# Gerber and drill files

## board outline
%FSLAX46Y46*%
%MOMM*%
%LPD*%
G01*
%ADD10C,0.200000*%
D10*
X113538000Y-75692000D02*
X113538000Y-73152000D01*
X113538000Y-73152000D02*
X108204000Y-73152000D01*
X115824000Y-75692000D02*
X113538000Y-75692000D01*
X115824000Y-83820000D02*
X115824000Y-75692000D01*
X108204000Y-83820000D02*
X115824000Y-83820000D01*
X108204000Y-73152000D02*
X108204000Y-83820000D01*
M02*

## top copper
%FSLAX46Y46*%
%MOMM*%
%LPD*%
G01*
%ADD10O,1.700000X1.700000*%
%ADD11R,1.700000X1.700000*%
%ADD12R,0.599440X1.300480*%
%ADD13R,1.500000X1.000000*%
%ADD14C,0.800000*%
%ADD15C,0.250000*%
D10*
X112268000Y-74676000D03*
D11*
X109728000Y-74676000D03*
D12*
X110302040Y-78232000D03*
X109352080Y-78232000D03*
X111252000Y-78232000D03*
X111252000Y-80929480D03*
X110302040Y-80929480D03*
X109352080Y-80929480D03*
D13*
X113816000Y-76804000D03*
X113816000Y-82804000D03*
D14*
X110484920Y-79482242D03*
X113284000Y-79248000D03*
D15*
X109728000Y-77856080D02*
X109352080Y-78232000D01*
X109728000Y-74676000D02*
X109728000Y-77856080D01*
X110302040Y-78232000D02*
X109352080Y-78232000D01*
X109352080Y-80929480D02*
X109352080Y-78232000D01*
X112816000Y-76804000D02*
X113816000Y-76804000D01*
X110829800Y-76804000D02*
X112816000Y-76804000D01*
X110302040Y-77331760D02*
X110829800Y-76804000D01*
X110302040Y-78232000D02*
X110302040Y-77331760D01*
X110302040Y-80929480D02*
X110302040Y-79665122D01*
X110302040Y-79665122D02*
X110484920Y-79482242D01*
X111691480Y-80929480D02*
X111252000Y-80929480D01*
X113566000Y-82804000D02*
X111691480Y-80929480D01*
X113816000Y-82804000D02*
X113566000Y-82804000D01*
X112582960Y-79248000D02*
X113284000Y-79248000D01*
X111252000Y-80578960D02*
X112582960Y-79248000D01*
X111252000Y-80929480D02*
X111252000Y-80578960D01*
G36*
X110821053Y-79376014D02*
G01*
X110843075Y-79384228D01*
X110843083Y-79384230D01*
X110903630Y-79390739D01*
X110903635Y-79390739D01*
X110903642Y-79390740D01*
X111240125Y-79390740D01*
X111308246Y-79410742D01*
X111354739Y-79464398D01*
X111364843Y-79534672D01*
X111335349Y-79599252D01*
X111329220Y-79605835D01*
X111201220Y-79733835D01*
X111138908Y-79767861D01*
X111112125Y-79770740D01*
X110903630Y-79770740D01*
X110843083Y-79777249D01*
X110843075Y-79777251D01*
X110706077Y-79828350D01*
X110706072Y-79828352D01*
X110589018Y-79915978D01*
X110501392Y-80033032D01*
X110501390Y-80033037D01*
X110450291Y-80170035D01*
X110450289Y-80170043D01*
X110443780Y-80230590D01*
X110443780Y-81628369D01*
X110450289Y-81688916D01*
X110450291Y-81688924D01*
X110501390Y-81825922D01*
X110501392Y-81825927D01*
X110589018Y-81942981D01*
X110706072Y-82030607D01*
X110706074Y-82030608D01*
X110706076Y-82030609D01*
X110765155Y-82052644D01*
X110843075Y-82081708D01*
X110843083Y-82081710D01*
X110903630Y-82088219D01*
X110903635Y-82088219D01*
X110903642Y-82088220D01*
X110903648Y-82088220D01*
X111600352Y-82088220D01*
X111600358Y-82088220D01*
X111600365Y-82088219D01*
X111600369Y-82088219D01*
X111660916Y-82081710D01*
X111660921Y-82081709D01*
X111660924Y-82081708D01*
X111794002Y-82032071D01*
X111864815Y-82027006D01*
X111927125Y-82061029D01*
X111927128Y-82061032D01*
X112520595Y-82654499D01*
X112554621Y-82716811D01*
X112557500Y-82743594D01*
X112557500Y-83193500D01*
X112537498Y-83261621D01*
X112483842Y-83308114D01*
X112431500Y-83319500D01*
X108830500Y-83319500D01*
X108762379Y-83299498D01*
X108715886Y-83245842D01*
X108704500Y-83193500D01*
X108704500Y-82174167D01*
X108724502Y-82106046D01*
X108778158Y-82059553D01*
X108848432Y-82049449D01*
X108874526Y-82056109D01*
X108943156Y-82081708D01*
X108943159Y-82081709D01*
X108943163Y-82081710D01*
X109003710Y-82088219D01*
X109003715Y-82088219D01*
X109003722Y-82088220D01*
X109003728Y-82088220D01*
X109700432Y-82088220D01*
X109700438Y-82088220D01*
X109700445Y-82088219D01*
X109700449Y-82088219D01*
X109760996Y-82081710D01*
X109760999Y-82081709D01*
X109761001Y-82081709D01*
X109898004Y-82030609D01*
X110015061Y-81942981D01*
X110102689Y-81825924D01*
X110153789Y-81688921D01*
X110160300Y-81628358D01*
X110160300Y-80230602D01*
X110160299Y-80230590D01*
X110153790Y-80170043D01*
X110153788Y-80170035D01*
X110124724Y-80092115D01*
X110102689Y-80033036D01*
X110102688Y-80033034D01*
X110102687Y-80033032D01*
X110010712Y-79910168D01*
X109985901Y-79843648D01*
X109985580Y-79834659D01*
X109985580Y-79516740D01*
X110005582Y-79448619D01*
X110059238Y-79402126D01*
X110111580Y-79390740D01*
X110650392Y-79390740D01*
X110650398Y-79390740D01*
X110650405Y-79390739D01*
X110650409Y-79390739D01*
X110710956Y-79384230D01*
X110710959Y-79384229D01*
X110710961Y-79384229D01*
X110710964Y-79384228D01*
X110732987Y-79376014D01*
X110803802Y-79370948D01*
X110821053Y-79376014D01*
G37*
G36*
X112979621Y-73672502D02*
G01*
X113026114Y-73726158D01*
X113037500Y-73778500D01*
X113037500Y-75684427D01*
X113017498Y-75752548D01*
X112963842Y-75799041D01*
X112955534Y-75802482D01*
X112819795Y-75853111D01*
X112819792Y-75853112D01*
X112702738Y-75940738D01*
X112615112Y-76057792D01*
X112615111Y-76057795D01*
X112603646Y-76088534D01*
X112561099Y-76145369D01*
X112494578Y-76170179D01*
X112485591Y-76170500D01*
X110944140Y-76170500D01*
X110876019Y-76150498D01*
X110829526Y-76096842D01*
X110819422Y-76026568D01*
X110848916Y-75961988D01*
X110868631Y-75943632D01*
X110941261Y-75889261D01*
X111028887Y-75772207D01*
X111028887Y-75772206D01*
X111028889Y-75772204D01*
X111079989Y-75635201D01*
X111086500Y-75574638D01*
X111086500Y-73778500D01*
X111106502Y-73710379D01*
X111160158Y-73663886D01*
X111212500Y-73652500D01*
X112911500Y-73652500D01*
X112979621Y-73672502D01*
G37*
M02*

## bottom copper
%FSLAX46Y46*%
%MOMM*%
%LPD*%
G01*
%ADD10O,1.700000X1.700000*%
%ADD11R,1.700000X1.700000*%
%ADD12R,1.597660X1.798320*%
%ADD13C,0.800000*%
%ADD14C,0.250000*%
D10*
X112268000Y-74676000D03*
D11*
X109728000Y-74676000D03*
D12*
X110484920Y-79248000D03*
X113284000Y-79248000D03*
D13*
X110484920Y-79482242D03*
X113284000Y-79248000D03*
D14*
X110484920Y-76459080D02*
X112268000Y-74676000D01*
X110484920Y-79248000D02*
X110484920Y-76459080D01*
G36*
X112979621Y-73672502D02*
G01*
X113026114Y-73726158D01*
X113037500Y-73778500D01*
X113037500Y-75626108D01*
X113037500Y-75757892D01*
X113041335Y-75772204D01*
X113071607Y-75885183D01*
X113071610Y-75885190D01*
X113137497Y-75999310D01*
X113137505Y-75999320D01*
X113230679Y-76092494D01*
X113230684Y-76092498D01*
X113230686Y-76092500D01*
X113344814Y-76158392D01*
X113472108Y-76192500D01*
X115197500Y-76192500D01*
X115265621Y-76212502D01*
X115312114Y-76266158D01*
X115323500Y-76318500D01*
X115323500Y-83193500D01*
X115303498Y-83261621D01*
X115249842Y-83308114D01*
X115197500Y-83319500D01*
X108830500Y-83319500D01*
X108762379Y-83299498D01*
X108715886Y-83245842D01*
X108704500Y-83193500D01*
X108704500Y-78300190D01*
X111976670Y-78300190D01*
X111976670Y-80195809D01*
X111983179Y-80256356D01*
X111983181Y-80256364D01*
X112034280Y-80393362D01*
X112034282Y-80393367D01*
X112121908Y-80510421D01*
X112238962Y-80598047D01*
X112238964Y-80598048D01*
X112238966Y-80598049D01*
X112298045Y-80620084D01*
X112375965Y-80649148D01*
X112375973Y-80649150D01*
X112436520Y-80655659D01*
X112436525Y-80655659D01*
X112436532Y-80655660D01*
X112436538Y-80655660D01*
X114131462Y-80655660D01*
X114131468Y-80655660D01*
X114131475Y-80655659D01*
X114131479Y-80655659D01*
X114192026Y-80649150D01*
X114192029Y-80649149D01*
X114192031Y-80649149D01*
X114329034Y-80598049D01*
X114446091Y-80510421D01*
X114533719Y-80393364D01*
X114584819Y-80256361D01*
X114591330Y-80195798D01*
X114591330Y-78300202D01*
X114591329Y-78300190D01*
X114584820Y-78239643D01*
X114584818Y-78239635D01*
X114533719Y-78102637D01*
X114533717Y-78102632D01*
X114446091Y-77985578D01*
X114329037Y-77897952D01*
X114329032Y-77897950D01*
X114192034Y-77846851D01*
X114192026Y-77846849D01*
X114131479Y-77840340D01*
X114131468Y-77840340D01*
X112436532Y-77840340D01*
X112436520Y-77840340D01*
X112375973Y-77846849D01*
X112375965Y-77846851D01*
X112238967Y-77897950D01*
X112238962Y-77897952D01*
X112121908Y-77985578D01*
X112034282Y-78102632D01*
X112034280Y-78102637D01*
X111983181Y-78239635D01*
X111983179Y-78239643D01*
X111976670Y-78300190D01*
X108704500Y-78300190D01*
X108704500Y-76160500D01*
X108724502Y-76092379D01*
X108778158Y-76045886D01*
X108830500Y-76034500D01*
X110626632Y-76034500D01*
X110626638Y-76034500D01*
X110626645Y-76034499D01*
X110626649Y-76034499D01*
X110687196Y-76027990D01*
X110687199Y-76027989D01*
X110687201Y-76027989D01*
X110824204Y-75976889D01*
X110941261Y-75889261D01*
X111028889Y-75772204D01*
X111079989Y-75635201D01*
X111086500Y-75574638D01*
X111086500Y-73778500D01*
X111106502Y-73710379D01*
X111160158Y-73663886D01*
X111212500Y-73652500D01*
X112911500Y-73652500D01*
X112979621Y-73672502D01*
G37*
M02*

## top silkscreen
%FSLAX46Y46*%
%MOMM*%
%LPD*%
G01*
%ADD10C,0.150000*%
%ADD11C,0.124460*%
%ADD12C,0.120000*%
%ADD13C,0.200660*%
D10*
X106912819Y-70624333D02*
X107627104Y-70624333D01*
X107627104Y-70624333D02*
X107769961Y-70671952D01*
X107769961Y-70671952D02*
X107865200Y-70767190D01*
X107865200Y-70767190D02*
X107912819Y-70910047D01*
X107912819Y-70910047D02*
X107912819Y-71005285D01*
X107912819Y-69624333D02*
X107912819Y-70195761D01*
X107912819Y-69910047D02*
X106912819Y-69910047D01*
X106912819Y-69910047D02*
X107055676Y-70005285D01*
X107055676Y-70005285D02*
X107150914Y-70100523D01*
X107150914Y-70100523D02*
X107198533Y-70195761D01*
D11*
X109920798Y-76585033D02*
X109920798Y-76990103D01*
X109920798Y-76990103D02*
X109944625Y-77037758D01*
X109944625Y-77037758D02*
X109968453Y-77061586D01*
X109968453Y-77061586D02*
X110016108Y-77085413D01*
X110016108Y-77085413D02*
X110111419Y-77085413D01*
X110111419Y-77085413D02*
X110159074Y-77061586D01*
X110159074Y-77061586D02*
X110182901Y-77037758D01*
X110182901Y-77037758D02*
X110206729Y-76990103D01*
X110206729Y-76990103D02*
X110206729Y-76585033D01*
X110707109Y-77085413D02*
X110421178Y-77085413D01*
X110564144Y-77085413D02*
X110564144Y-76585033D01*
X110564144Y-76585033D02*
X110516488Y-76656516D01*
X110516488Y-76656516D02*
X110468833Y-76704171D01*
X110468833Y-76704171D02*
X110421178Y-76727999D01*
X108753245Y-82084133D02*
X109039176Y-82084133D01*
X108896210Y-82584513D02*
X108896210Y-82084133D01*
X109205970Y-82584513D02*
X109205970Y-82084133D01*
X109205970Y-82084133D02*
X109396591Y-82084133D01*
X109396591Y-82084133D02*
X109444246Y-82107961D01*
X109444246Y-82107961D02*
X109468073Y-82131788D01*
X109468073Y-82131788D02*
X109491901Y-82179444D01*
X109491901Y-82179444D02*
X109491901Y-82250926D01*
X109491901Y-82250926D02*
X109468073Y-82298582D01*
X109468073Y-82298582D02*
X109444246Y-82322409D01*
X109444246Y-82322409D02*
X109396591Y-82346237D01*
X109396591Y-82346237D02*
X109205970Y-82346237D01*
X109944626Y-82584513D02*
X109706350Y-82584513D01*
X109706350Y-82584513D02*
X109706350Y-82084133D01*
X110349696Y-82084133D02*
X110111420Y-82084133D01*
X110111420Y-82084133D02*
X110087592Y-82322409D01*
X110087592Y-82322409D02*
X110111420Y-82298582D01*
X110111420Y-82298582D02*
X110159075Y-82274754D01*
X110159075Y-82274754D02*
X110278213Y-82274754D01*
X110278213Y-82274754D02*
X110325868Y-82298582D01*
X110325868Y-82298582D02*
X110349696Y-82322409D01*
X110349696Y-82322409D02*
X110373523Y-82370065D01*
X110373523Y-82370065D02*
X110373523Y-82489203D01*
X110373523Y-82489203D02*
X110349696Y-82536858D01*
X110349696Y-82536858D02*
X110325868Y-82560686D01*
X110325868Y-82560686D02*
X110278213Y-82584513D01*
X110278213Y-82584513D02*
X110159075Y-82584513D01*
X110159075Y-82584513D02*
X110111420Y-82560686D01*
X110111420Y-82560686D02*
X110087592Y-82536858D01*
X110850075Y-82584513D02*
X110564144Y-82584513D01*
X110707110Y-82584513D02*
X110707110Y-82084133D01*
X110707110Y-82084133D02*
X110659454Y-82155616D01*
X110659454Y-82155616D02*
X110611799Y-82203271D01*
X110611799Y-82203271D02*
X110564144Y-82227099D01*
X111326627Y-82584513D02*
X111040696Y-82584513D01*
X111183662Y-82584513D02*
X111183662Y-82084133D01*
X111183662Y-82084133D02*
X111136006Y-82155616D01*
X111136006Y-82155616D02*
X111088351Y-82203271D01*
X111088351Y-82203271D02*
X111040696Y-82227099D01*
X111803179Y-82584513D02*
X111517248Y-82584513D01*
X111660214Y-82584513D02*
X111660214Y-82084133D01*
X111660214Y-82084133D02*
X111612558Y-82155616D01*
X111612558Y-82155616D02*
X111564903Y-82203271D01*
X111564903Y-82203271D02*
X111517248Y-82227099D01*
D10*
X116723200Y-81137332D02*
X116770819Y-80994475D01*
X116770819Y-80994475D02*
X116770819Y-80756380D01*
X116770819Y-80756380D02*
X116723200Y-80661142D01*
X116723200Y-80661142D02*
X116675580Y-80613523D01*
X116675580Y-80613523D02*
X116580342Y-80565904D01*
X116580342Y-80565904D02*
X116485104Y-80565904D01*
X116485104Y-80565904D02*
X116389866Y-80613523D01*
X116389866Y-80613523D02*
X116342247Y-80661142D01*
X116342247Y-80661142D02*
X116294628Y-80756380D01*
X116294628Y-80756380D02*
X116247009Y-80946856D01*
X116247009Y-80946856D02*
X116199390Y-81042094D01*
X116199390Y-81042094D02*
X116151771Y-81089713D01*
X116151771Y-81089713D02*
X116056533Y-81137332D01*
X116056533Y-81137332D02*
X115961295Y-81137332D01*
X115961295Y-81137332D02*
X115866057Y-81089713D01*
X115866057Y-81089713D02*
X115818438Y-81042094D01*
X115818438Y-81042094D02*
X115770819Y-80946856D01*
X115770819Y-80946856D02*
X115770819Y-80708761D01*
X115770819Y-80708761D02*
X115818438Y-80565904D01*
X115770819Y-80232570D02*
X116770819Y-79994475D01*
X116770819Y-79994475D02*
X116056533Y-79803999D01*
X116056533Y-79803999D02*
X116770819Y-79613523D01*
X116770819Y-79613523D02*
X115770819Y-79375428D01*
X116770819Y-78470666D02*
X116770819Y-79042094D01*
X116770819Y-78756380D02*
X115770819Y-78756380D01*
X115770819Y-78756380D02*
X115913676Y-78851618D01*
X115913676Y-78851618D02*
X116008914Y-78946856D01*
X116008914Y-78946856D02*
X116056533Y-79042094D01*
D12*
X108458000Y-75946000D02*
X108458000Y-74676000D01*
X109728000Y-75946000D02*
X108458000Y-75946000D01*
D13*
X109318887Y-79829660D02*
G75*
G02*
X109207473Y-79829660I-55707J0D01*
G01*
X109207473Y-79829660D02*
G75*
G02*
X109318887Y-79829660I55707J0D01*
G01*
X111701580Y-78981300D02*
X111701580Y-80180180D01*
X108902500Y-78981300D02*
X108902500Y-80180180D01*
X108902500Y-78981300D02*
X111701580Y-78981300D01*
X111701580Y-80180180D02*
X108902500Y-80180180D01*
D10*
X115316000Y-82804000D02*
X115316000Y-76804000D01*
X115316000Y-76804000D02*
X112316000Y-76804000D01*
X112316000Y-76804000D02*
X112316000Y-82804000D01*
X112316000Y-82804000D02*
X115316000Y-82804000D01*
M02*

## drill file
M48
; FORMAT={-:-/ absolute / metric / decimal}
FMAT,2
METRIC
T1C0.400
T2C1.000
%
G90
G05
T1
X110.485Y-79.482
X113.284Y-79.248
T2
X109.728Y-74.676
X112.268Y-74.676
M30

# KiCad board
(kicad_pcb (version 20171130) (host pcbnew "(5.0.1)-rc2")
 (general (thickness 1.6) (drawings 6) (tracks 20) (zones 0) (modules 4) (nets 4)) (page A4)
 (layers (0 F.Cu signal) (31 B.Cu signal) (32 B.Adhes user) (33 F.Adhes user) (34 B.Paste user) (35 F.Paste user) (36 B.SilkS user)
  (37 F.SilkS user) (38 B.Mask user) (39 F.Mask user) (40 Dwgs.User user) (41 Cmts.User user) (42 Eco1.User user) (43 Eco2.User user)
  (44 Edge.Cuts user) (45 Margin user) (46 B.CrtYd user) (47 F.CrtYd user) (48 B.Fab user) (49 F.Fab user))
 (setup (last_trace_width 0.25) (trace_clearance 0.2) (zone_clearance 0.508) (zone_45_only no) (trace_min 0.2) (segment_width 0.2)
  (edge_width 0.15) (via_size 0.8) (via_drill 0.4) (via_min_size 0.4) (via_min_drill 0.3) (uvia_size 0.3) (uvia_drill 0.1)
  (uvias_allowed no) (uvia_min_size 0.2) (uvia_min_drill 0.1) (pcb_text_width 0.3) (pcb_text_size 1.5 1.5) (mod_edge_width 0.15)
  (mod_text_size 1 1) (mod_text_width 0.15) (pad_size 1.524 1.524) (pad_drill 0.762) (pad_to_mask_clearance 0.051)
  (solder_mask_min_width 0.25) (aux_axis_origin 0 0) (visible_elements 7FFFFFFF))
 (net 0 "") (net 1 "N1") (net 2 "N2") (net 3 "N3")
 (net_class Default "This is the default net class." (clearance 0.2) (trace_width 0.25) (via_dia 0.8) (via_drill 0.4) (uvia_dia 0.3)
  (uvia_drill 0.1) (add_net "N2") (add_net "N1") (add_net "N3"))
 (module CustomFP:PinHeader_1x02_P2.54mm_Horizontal (layer F.Cu) (at 109.728 74.676 90)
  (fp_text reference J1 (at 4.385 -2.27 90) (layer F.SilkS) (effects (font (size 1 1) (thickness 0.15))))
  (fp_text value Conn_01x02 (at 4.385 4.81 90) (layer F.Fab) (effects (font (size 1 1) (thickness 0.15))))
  (fp_line (start -1.27 -1.27) (end 0 -1.27) (layer F.SilkS) (width 0.12))
  (fp_line (start -1.27 0) (end -1.27 -1.27) (layer F.SilkS) (width 0.12))
  (pad 2 thru_hole oval (at 0 2.54 90) (size 1.7 1.7) (drill 1) (layers *.Cu *.Mask) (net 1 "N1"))
  (pad 1 thru_hole rect (at 0 0 90) (size 1.7 1.7) (drill 1) (layers *.Cu *.Mask) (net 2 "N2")))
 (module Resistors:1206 (layer B.Cu) (at 111.88446 79.248)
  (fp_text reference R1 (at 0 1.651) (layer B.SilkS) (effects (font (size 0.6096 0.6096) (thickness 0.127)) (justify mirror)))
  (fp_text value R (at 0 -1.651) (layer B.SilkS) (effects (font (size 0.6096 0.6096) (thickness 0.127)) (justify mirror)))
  (pad 1 smd rect (at -1.39954 0) (size 1.59766 1.79832) (layers B.Cu B.Paste B.Mask) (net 1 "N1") (solder_mask_margin 0.1016))
  (pad 2 smd rect (at 1.39954 0) (size 1.59766 1.79832) (layers B.Cu B.Paste B.Mask) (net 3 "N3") (solder_mask_margin 0.1016)))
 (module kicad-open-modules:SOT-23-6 (layer F.Cu) (at 110.30204 79.58074)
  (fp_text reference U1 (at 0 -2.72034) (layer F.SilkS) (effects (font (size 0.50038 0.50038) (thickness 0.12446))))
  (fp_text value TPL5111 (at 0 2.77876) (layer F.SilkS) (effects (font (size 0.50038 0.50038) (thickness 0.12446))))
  (fp_circle (center -1.03886 0.24892) (end -1.00076 0.28956) (layer F.SilkS) (width 0.20066))
  (fp_line (start 1.39954 -0.59944) (end 1.39954 0.59944) (layer F.SilkS) (width 0.20066))
  (fp_line (start -1.39954 -0.59944) (end -1.39954 0.59944) (layer F.SilkS) (width 0.20066))
  (fp_line (start -1.39954 -0.59944) (end 1.39954 -0.59944) (layer F.SilkS) (width 0.20066))
  (fp_line (start 1.39954 0.59944) (end -1.39954 0.59944) (layer F.SilkS) (width 0.20066))
  (pad 5 smd rect (at 0 -1.34874) (size 0.59944 1.30048) (layers F.Cu F.Paste F.Mask) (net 2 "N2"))
  (pad 6 smd rect (at -0.94996 -1.34874) (size 0.59944 1.30048) (layers F.Cu F.Paste F.Mask) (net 2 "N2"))
  (pad 4 smd rect (at 0.94996 -1.34874) (size 0.59944 1.30048) (layers F.Cu F.Paste F.Mask))
  (pad 3 smd rect (at 0.94996 1.34874) (size 0.59944 1.30048) (layers F.Cu F.Paste F.Mask) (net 3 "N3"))
  (pad 2 smd rect (at 0 1.34874) (size 0.59944 1.30048) (layers F.Cu F.Paste F.Mask) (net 1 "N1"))
  (pad 1 smd rect (at -0.94996 1.34874) (size 0.59944 1.30048) (layers F.Cu F.Paste F.Mask) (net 2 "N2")))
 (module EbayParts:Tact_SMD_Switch (layer F.Cu) (at 115.316 82.804 90)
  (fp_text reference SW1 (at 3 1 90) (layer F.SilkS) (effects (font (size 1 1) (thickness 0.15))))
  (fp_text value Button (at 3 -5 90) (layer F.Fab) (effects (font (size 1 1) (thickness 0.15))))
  (fp_line (start 0 0) (end 6 0) (layer F.SilkS) (width 0.15))
  (fp_line (start 6 0) (end 6 -3) (layer F.SilkS) (width 0.15))
  (fp_line (start 6 -3) (end 0 -3) (layer F.SilkS) (width 0.15))
  (fp_line (start 0 -3) (end 0 0) (layer F.SilkS) (width 0.15))
  (pad 2 smd rect (at 6 -1.5 90) (size 1 1.5) (layers F.Cu F.Paste F.Mask) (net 2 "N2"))
  (pad 1 smd rect (at 0 -1.5 90) (size 1 1.5) (layers F.Cu F.Paste F.Mask) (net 3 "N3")))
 (gr_line (start 113.538 75.692) (end 113.538 73.152) (layer Edge.Cuts) (width 0.2))
 (gr_line (start 113.538 73.152) (end 108.204 73.152) (layer Edge.Cuts) (width 0.2))
 (gr_line (start 115.824 75.692) (end 113.538 75.692) (layer Edge.Cuts) (width 0.2))
 (gr_line (start 115.824 83.82) (end 115.824 75.692) (layer Edge.Cuts) (width 0.2))
 (gr_line (start 108.204 83.82) (end 115.824 83.82) (layer Edge.Cuts) (width 0.2))
 (gr_line (start 108.204 73.152) (end 108.204 83.82) (layer Edge.Cuts) (width 0.2))
 (segment (start 109.728 77.85608) (end 109.35208 78.232) (width 0.25) (layer F.Cu) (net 2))
 (segment (start 109.728 74.676) (end 109.728 77.85608) (width 0.25) (layer F.Cu) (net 2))
 (segment (start 110.30204 78.232) (end 109.35208 78.232) (width 0.25) (layer F.Cu) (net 2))
 (segment (start 109.35208 80.92948) (end 109.35208 78.232) (width 0.25) (layer F.Cu) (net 2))
 (segment (start 112.816 76.804) (end 113.816 76.804) (width 0.25) (layer F.Cu) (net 2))
 (segment (start 110.8298 76.804) (end 112.816 76.804) (width 0.25) (layer F.Cu) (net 2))
 (segment (start 110.30204 77.33176) (end 110.8298 76.804) (width 0.25) (layer F.Cu) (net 2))
 (segment (start 110.30204 78.232) (end 110.30204 77.33176) (width 0.25) (layer F.Cu) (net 2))
 (via (at 110.48492 79.482242) (size 0.8) (drill 0.4) (layers F.Cu B.Cu) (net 1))
 (segment (start 110.30204 80.92948) (end 110.30204 79.665122) (width 0.25) (layer F.Cu) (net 1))
 (segment (start 110.30204 79.665122) (end 110.48492 79.482242) (width 0.25) (layer F.Cu) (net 1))
 (segment (start 110.48492 76.45908) (end 112.268 74.676) (width 0.25) (layer B.Cu) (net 1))
 (segment (start 110.48492 79.248) (end 110.48492 76.45908) (width 0.25) (layer B.Cu) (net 1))
 (segment (start 111.69148 80.92948) (end 111.252 80.92948) (width 0.25) (layer F.Cu) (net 3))
 (segment (start 113.566 82.804) (end 111.69148 80.92948) (width 0.25) (layer F.Cu) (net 3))
 (segment (start 113.816 82.804) (end 113.566 82.804) (width 0.25) (layer F.Cu) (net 3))
 (via (at 113.284 79.248) (size 0.8) (drill 0.4) (layers F.Cu B.Cu) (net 3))
 (segment (start 112.58296 79.248) (end 113.284 79.248) (width 0.25) (layer F.Cu) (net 3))
 (segment (start 111.252 80.57896) (end 112.58296 79.248) (width 0.25) (layer F.Cu) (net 3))
 (segment (start 111.252 80.92948) (end 111.252 80.57896) (width 0.25) (layer F.Cu) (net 3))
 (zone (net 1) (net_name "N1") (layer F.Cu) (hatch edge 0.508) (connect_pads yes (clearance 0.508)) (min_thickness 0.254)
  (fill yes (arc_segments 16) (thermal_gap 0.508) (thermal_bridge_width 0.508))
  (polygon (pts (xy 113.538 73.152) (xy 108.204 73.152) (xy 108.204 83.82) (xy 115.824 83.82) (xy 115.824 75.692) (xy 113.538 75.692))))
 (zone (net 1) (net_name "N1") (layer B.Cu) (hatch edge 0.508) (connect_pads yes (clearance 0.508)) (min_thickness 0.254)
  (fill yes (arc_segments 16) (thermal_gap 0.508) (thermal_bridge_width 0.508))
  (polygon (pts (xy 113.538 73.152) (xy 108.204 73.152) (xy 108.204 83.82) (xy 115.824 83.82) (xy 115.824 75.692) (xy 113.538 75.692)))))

